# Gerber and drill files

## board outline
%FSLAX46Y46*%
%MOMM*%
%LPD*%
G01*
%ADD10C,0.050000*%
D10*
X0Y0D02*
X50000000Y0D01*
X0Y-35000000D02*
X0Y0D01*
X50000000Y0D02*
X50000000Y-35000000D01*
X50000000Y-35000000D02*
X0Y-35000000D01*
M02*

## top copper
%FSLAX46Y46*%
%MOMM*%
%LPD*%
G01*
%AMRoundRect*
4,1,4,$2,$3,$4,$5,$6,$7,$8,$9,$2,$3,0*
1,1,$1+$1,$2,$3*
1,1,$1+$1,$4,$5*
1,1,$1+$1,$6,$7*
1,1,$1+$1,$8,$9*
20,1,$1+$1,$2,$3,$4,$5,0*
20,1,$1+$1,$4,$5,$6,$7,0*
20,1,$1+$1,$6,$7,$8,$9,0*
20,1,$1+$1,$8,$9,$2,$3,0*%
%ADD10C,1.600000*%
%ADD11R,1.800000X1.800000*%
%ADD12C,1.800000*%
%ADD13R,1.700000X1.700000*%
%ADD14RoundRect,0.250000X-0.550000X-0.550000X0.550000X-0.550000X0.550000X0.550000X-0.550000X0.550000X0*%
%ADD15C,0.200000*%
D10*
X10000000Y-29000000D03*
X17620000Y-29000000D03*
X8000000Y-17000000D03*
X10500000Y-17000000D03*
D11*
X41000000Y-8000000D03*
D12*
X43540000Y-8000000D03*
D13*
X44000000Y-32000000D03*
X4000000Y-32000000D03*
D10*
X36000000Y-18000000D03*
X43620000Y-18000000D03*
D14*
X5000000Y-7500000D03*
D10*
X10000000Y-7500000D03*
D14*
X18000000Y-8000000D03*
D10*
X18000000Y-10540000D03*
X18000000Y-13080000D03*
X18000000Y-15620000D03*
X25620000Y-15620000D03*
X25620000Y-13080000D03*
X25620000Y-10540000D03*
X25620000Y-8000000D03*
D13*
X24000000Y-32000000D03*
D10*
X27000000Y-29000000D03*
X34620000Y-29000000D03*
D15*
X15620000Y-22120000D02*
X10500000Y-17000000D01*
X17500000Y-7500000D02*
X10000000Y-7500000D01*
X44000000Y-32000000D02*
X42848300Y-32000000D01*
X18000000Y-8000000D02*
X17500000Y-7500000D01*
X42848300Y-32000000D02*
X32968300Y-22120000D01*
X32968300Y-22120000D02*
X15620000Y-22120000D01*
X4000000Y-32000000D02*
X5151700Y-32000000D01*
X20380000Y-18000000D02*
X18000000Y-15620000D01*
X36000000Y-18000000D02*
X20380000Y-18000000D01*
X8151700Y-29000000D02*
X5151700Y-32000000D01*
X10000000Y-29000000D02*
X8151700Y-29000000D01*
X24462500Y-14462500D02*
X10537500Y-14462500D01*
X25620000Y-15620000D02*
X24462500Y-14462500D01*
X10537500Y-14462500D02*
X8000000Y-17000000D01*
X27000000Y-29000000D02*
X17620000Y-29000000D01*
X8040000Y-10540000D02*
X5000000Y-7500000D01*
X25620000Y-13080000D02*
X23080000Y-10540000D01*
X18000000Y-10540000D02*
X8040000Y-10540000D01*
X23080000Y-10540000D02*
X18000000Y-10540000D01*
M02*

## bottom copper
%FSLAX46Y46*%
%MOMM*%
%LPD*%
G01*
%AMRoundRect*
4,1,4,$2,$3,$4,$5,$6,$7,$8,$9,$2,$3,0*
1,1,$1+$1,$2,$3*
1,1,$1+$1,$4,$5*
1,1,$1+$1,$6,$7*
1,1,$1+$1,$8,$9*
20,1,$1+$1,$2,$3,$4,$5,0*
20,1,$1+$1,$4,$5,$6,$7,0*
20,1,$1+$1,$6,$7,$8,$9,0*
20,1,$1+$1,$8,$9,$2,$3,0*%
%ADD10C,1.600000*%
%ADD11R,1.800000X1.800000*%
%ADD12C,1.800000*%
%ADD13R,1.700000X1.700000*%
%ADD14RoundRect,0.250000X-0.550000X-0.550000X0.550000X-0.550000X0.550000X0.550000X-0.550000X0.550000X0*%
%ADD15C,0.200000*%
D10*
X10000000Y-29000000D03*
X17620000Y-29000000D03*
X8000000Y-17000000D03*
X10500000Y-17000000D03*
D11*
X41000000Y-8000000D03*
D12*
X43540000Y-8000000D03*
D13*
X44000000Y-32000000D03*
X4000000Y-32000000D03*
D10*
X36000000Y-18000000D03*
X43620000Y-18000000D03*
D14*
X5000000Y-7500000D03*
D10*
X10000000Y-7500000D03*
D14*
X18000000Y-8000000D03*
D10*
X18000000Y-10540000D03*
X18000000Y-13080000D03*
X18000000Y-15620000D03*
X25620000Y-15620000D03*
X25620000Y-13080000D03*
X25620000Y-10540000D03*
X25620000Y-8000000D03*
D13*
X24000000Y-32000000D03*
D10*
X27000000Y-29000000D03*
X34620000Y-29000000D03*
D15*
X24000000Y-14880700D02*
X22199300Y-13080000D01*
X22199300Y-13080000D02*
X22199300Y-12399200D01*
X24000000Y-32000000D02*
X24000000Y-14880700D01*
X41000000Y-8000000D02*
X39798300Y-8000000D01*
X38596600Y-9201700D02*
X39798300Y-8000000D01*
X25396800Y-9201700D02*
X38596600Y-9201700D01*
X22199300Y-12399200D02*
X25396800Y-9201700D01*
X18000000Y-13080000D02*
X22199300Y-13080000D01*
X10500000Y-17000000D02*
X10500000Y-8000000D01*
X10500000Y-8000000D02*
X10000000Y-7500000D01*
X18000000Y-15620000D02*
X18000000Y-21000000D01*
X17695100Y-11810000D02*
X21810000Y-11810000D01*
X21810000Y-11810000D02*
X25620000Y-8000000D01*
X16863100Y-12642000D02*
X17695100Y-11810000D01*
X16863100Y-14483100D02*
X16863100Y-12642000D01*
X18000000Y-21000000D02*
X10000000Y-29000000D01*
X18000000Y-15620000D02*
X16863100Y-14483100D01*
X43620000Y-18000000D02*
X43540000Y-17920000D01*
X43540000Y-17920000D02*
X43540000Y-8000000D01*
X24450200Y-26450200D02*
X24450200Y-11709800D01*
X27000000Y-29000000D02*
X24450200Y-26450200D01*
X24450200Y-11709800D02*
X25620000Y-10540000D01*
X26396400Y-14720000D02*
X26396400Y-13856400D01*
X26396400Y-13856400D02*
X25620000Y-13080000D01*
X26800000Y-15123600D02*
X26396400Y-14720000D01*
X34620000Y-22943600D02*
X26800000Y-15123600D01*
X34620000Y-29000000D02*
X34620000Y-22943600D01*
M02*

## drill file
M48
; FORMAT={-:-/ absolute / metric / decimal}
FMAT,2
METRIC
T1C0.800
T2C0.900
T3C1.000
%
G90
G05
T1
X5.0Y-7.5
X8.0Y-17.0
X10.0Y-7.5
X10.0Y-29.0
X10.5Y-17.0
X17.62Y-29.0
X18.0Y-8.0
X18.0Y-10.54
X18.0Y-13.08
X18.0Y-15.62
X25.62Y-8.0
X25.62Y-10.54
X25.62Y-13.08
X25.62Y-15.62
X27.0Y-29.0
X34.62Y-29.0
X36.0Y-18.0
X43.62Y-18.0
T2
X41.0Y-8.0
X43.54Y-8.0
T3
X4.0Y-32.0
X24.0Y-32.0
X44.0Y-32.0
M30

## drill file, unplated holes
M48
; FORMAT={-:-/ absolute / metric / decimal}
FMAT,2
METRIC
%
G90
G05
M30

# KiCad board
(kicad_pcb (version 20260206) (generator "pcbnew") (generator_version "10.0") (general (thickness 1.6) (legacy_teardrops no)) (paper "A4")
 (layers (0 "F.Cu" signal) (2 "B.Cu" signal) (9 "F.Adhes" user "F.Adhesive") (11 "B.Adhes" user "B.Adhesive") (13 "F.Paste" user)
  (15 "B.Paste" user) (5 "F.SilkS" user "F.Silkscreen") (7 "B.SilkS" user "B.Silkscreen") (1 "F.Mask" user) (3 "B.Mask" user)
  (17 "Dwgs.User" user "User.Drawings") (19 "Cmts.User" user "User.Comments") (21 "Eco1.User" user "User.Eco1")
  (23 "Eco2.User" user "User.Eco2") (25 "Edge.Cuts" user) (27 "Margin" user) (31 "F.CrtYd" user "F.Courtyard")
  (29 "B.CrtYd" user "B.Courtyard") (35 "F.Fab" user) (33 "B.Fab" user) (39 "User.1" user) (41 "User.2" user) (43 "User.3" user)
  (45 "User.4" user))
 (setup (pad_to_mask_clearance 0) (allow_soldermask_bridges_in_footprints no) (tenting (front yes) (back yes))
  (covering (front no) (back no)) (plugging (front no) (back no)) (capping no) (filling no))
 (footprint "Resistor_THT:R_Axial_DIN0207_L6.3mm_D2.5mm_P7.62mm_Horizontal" (layer "F.Cu") (at 10 29)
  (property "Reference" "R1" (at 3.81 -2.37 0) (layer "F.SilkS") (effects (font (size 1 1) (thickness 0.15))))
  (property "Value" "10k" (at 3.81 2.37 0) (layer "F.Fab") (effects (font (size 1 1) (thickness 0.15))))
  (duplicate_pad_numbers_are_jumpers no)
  (pad "1" thru_hole circle (at 0 0) (size 1.6 1.6) (drill 0.8) (layers "*.Cu" "*.Mask") (remove_unused_layers no) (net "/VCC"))
  (pad "2" thru_hole circle (at 7.62 0) (size 1.6 1.6) (drill 0.8) (layers "*.Cu" "*.Mask") (remove_unused_layers no) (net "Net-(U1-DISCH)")))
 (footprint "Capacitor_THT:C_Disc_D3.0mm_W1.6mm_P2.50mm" (layer "F.Cu") (at 8 17)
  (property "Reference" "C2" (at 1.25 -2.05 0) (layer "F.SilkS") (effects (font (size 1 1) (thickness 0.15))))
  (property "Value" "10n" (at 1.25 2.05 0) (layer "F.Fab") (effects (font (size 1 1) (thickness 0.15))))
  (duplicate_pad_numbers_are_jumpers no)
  (pad "1" thru_hole circle (at 0 0) (size 1.6 1.6) (drill 0.8) (layers "*.Cu" "*.Mask") (remove_unused_layers no) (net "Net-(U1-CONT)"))
  (pad "2" thru_hole circle (at 2.5 0) (size 1.6 1.6) (drill 0.8) (layers "*.Cu" "*.Mask") (remove_unused_layers no) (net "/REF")))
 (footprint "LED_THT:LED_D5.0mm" (layer "F.Cu") (at 41 8)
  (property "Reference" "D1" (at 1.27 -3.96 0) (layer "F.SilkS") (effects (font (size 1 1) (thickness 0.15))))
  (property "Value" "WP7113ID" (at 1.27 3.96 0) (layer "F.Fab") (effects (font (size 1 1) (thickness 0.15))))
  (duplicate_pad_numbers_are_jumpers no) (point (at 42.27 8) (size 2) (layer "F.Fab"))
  (pad "1" thru_hole rect (at 0 0) (size 1.8 1.8) (drill 0.9) (layers "*.Cu" "*.Mask") (remove_unused_layers no) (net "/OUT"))
  (pad "2" thru_hole circle (at 2.54 0) (size 1.8 1.8) (drill 0.9) (layers "*.Cu" "*.Mask") (remove_unused_layers no) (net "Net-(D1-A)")))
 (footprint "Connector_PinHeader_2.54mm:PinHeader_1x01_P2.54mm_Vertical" (layer "F.Cu") (at 44 32)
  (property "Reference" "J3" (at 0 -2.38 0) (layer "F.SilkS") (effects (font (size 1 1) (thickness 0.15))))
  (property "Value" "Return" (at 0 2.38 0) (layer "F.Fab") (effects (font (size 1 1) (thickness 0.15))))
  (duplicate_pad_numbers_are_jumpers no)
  (pad "1" thru_hole rect (at 0 0) (size 1.7 1.7) (drill 1) (layers "*.Cu" "*.Mask") (remove_unused_layers no) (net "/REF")))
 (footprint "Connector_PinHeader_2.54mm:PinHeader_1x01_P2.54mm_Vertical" (layer "F.Cu") (at 4 32)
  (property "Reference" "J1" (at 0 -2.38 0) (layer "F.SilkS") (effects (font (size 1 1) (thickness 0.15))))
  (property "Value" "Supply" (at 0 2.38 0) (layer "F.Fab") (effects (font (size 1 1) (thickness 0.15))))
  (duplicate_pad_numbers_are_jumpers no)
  (pad "1" thru_hole rect (at 0 0) (size 1.7 1.7) (drill 1) (layers "*.Cu" "*.Mask") (remove_unused_layers no) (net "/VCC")))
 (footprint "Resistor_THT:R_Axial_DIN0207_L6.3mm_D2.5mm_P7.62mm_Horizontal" (layer "F.Cu") (at 36 18)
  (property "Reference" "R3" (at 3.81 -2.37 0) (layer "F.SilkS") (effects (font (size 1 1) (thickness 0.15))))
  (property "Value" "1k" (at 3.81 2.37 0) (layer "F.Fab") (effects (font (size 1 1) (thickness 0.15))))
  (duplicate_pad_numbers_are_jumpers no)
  (pad "1" thru_hole circle (at 0 0) (size 1.6 1.6) (drill 0.8) (layers "*.Cu" "*.Mask") (remove_unused_layers no) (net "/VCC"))
  (pad "2" thru_hole circle (at 7.62 0) (size 1.6 1.6) (drill 0.8) (layers "*.Cu" "*.Mask") (remove_unused_layers no) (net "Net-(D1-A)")))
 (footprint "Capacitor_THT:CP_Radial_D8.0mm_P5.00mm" (layer "F.Cu") (at 5 7.5)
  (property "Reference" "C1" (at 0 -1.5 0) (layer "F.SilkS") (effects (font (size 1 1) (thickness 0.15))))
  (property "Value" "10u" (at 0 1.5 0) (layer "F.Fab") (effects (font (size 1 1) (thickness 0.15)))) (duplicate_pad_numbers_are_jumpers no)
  (pad "1" thru_hole roundrect (at 0 0) (size 1.6 1.6) (drill 0.8) (layers "*.Cu" "*.Mask") (remove_unused_layers no)
   (roundrect_rratio 0.15625) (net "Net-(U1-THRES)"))
  (pad "2" thru_hole circle (at 5 0) (size 1.6 1.6) (drill 0.8) (layers "*.Cu" "*.Mask") (remove_unused_layers no) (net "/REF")))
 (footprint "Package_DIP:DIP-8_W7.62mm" (layer "F.Cu") (at 18 8)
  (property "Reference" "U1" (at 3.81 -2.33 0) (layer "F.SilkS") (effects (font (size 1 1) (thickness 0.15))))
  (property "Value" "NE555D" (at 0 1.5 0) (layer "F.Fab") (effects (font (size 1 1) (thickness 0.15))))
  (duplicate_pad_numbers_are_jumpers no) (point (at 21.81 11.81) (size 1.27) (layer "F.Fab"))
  (pad "1" thru_hole roundrect (at 0 0) (size 1.6 1.6) (drill 0.8) (layers "*.Cu" "*.Mask") (remove_unused_layers no)
   (roundrect_rratio 0.15625) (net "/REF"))
  (pad "2" thru_hole circle (at 0 2.54) (size 1.6 1.6) (drill 0.8) (layers "*.Cu" "*.Mask") (remove_unused_layers no) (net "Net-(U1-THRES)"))
  (pad "3" thru_hole circle (at 0 5.08) (size 1.6 1.6) (drill 0.8) (layers "*.Cu" "*.Mask") (remove_unused_layers no) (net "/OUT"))
  (pad "4" thru_hole circle (at 0 7.62) (size 1.6 1.6) (drill 0.8) (layers "*.Cu" "*.Mask") (remove_unused_layers no) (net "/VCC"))
  (pad "5" thru_hole circle (at 7.62 7.62) (size 1.6 1.6) (drill 0.8) (layers "*.Cu" "*.Mask") (remove_unused_layers no)
   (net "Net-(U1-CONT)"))
  (pad "6" thru_hole circle (at 7.62 5.08) (size 1.6 1.6) (drill 0.8) (layers "*.Cu" "*.Mask") (remove_unused_layers no)
   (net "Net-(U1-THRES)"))
  (pad "7" thru_hole circle (at 7.62 2.54) (size 1.6 1.6) (drill 0.8) (layers "*.Cu" "*.Mask") (remove_unused_layers no)
   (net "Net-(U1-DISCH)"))
  (pad "8" thru_hole circle (at 7.62 0) (size 1.6 1.6) (drill 0.8) (layers "*.Cu" "*.Mask") (remove_unused_layers no) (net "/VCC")))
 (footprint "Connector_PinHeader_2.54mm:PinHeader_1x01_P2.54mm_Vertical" (layer "F.Cu") (at 24 32)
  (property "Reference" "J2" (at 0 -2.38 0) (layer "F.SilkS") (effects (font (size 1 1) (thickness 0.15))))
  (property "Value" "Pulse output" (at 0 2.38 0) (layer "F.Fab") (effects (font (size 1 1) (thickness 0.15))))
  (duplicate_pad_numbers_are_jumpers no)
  (pad "1" thru_hole rect (at 0 0) (size 1.7 1.7) (drill 1) (layers "*.Cu" "*.Mask") (remove_unused_layers no) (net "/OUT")))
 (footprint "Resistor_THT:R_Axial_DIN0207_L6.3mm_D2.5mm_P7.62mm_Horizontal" (layer "F.Cu") (at 27 29)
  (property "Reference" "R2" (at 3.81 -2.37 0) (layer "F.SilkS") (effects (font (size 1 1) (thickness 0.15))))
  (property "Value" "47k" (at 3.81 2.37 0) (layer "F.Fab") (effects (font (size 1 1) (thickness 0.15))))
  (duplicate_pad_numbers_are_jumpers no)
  (pad "1" thru_hole circle (at 0 0) (size 1.6 1.6) (drill 0.8) (layers "*.Cu" "*.Mask") (remove_unused_layers no) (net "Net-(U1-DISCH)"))
  (pad "2" thru_hole circle (at 7.62 0) (size 1.6 1.6) (drill 0.8) (layers "*.Cu" "*.Mask") (remove_unused_layers no) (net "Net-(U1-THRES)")))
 (gr_line (start 0 0) (end 50 0) (stroke (width 0.05) (type default)) (layer "Edge.Cuts"))
 (gr_line (start 0 35) (end 0 0) (stroke (width 0.05) (type default)) (layer "Edge.Cuts"))
 (gr_line (start 50 0) (end 50 35) (stroke (width 0.05) (type default)) (layer "Edge.Cuts"))
 (gr_line (start 50 35) (end 0 35) (stroke (width 0.05) (type default)) (layer "Edge.Cuts"))
 (segment (start 4 32) (end 5.1517 32) (width 0.2) (layer "F.Cu") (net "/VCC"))
 (segment (start 20.38 18) (end 18 15.62) (width 0.2) (layer "F.Cu") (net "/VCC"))
 (segment (start 36 18) (end 20.38 18) (width 0.2) (layer "F.Cu") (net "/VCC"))
 (segment (start 8.1517 29) (end 5.1517 32) (width 0.2) (layer "F.Cu") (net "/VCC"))
 (segment (start 10 29) (end 8.1517 29) (width 0.2) (layer "F.Cu") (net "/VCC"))
 (segment (start 18 15.62) (end 18 21) (width 0.2) (layer "B.Cu") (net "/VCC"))
 (segment (start 17.6951 11.81) (end 21.81 11.81) (width 0.2) (layer "B.Cu") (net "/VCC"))
 (segment (start 21.81 11.81) (end 25.62 8) (width 0.2) (layer "B.Cu") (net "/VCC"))
 (segment (start 16.8631 12.642) (end 17.6951 11.81) (width 0.2) (layer "B.Cu") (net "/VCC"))
 (segment (start 16.8631 14.4831) (end 16.8631 12.642) (width 0.2) (layer "B.Cu") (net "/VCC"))
 (segment (start 18 21) (end 10 29) (width 0.2) (layer "B.Cu") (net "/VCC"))
 (segment (start 18 15.62) (end 16.8631 14.4831) (width 0.2) (layer "B.Cu") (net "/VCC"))
 (segment (start 27 29) (end 17.62 29) (width 0.2) (layer "F.Cu") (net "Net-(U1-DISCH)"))
 (segment (start 24.4502 26.4502) (end 24.4502 11.7098) (width 0.2) (layer "B.Cu") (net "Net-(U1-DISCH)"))
 (segment (start 27 29) (end 24.4502 26.4502) (width 0.2) (layer "B.Cu") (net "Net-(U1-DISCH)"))
 (segment (start 24.4502 11.7098) (end 25.62 10.54) (width 0.2) (layer "B.Cu") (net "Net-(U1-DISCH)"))
 (segment (start 24.4625 14.4625) (end 10.5375 14.4625) (width 0.2) (layer "F.Cu") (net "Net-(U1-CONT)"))
 (segment (start 25.62 15.62) (end 24.4625 14.4625) (width 0.2) (layer "F.Cu") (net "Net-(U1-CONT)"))
 (segment (start 10.5375 14.4625) (end 8 17) (width 0.2) (layer "F.Cu") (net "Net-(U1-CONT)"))
 (segment (start 15.62 22.12) (end 10.5 17) (width 0.2) (layer "F.Cu") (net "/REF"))
 (segment (start 17.5 7.5) (end 10 7.5) (width 0.2) (layer "F.Cu") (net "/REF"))
 (segment (start 44 32) (end 42.8483 32) (width 0.2) (layer "F.Cu") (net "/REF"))
 (segment (start 18 8) (end 17.5 7.5) (width 0.2) (layer "F.Cu") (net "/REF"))
 (segment (start 42.8483 32) (end 32.9683 22.12) (width 0.2) (layer "F.Cu") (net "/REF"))
 (segment (start 32.9683 22.12) (end 15.62 22.12) (width 0.2) (layer "F.Cu") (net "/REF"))
 (segment (start 10.5 17) (end 10.5 8) (width 0.2) (layer "B.Cu") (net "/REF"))
 (segment (start 10.5 8) (end 10 7.5) (width 0.2) (layer "B.Cu") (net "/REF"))
 (segment (start 24 14.8807) (end 22.1993 13.08) (width 0.2) (layer "B.Cu") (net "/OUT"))
 (segment (start 22.1993 13.08) (end 22.1993 12.3992) (width 0.2) (layer "B.Cu") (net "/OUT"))
 (segment (start 24 32) (end 24 14.8807) (width 0.2) (layer "B.Cu") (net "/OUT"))
 (segment (start 41 8) (end 39.7983 8) (width 0.2) (layer "B.Cu") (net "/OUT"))
 (segment (start 38.5966 9.2017) (end 39.7983 8) (width 0.2) (layer "B.Cu") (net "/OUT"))
 (segment (start 25.3968 9.2017) (end 38.5966 9.2017) (width 0.2) (layer "B.Cu") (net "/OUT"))
 (segment (start 22.1993 12.3992) (end 25.3968 9.2017) (width 0.2) (layer "B.Cu") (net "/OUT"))
 (segment (start 18 13.08) (end 22.1993 13.08) (width 0.2) (layer "B.Cu") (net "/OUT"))
 (segment (start 43.62 18) (end 43.54 17.92) (width 0.2) (layer "B.Cu") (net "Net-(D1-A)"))
 (segment (start 43.54 17.92) (end 43.54 8) (width 0.2) (layer "B.Cu") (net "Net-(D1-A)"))
 (segment (start 8.04 10.54) (end 5 7.5) (width 0.2) (layer "F.Cu") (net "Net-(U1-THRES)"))
 (segment (start 25.62 13.08) (end 23.08 10.54) (width 0.2) (layer "F.Cu") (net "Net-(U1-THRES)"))
 (segment (start 18 10.54) (end 8.04 10.54) (width 0.2) (layer "F.Cu") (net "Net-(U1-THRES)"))
 (segment (start 23.08 10.54) (end 18 10.54) (width 0.2) (layer "F.Cu") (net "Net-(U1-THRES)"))
 (segment (start 26.3964 14.72) (end 26.3964 13.8564) (width 0.2) (layer "B.Cu") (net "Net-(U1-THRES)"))
 (segment (start 26.3964 13.8564) (end 25.62 13.08) (width 0.2) (layer "B.Cu") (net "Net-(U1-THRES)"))
 (segment (start 26.8 15.1236) (end 26.3964 14.72) (width 0.2) (layer "B.Cu") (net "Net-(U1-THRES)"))
 (segment (start 34.62 22.9436) (end 26.8 15.1236) (width 0.2) (layer "B.Cu") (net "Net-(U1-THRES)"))
 (segment (start 34.62 29) (end 34.62 22.9436) (width 0.2) (layer "B.Cu") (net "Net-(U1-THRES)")))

